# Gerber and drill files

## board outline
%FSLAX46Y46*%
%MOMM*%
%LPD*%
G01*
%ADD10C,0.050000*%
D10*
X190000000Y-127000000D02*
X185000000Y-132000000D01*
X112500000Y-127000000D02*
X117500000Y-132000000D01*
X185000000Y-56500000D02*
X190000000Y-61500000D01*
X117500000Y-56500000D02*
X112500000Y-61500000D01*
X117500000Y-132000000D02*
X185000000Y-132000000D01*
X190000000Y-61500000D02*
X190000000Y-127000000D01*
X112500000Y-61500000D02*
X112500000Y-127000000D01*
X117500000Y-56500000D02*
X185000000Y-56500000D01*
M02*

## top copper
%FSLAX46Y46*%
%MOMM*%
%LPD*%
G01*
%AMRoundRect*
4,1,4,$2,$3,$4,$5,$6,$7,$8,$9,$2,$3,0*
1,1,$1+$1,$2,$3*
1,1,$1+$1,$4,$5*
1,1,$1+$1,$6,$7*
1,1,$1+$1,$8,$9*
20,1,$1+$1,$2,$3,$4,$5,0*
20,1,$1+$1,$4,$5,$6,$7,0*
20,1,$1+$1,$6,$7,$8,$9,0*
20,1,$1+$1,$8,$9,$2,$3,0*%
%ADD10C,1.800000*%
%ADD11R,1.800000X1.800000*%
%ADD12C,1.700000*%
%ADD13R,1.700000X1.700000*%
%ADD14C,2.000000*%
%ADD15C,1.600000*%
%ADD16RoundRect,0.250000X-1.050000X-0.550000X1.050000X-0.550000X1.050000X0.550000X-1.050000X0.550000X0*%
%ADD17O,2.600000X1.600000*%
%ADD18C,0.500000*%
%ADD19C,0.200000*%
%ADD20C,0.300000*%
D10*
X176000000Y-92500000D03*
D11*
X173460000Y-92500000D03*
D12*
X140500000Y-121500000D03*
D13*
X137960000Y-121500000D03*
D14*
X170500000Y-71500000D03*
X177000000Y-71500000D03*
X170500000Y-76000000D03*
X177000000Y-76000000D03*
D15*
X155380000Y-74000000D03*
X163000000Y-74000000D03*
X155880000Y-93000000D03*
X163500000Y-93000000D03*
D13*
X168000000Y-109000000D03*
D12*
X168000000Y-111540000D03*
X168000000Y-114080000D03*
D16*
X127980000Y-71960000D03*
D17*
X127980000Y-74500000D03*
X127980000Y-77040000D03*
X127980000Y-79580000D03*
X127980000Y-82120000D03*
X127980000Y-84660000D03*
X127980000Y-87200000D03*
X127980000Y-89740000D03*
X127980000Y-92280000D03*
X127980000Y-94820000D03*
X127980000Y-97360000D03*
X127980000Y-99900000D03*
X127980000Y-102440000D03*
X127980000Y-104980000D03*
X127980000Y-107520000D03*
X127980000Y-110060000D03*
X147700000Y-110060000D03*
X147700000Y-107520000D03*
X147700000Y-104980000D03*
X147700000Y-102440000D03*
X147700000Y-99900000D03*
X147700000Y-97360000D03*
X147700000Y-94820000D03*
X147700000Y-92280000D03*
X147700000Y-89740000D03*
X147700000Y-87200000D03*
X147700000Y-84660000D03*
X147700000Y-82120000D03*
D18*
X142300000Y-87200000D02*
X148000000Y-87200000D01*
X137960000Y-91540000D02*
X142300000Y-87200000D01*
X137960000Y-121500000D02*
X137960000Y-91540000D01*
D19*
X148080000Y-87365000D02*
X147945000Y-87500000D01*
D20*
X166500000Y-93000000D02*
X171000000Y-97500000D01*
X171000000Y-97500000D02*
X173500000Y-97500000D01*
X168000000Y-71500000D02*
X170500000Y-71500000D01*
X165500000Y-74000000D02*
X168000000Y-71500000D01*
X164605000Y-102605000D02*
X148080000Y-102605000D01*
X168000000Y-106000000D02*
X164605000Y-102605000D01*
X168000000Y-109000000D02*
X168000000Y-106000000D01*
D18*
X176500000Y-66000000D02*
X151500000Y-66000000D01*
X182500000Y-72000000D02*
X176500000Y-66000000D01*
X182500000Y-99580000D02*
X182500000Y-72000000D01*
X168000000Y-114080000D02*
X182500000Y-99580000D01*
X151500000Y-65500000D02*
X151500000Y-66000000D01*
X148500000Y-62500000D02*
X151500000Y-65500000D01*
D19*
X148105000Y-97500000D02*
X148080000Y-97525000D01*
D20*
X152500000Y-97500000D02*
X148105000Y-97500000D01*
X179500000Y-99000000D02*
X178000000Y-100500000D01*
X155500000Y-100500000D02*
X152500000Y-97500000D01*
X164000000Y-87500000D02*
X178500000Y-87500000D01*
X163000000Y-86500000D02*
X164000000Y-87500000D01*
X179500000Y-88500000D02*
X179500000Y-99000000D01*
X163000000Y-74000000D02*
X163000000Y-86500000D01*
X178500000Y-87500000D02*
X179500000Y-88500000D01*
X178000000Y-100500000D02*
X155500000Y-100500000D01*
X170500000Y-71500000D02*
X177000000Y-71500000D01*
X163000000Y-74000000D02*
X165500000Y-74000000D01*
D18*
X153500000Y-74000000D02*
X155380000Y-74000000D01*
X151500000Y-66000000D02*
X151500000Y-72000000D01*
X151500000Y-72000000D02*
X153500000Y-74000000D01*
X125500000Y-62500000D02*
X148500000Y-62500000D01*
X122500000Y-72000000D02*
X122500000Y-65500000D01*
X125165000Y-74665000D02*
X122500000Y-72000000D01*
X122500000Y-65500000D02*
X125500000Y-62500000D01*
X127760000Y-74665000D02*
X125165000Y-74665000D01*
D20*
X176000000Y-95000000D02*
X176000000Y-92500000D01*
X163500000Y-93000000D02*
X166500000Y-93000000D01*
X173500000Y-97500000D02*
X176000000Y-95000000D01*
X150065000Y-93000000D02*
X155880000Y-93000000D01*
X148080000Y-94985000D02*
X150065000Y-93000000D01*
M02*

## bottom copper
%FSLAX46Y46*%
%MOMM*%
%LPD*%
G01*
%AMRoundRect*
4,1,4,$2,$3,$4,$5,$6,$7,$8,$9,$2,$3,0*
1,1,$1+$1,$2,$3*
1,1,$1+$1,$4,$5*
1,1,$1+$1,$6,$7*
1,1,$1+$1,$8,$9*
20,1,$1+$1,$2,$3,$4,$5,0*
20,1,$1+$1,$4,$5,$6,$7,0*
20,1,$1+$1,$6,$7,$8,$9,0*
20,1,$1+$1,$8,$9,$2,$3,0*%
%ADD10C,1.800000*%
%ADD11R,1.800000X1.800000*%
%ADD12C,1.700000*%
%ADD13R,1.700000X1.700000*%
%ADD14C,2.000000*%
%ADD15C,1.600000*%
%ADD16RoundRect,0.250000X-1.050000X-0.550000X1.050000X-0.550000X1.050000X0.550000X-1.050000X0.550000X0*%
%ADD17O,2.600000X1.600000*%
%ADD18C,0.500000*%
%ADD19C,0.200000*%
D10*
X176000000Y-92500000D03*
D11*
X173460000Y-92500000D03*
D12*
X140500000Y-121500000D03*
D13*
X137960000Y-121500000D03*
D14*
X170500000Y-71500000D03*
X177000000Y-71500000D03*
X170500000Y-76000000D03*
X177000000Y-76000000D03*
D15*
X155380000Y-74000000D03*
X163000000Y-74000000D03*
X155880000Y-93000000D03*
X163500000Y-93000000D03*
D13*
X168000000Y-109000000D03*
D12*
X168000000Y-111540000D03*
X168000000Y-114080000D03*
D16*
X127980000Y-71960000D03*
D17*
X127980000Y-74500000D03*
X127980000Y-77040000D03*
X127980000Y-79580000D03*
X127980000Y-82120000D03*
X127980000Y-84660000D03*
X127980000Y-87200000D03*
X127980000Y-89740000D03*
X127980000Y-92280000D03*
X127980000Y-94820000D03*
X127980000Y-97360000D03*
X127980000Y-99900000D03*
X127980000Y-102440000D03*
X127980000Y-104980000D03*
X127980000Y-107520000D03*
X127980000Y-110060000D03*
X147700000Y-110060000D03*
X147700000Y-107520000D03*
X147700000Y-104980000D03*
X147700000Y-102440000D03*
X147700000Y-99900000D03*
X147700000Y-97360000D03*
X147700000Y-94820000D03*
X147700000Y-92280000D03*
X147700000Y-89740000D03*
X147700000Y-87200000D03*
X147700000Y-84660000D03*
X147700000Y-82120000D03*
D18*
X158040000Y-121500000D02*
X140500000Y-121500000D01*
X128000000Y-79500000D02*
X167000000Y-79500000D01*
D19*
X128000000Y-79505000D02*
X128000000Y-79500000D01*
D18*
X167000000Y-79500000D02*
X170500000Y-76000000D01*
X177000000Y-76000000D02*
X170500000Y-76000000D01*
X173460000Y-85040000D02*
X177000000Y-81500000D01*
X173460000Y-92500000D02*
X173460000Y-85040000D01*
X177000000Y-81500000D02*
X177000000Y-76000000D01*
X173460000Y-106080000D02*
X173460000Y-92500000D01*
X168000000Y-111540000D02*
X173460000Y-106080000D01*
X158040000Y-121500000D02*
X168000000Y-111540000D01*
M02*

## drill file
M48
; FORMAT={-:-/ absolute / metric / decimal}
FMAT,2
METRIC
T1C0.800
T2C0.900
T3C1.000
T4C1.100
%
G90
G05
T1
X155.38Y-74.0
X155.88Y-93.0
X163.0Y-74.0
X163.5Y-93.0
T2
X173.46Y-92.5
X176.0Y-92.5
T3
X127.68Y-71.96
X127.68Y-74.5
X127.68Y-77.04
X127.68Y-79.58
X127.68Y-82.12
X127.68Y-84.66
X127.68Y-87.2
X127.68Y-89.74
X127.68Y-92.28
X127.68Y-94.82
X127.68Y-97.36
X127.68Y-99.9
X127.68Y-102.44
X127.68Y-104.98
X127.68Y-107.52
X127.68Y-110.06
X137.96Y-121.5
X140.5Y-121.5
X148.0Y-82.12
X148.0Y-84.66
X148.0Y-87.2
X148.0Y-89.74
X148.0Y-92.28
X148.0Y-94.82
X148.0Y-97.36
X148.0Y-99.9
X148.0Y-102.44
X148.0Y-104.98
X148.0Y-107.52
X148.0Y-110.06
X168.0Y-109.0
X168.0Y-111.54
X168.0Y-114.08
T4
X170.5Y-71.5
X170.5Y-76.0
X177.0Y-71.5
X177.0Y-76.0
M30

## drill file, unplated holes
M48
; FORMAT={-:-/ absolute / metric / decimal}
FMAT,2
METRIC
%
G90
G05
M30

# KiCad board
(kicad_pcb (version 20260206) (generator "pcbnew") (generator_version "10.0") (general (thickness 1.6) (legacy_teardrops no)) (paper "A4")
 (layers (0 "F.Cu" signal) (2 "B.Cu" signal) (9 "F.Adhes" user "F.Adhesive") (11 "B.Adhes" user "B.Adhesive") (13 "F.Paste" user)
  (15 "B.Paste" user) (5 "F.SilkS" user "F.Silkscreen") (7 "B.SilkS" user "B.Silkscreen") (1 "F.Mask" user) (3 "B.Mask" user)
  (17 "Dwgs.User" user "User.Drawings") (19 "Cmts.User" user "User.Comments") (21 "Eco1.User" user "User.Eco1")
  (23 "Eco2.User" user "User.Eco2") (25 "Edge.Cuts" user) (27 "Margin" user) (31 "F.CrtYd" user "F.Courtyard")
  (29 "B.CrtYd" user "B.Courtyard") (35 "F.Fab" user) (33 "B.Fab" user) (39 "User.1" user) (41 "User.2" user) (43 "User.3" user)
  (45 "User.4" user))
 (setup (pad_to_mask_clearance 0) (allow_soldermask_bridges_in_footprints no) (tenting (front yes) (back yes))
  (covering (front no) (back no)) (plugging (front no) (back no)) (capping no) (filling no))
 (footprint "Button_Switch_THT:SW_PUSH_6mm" (layer "F.Cu") (at 170.5 71.5)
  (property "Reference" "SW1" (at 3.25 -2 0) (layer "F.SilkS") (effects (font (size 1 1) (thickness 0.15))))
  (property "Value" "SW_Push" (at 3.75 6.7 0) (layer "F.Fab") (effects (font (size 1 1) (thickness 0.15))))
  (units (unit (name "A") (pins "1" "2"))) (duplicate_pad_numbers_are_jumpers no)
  (pad "1" thru_hole circle (at 0 0 90) (size 2 2) (drill 1.1) (layers "*.Cu" "*.Mask") (remove_unused_layers no)
   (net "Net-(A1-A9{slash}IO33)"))
  (pad "1" thru_hole circle (at 6.5 0 90) (size 2 2) (drill 1.1) (layers "*.Cu" "*.Mask") (remove_unused_layers no)
   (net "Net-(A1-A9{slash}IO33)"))
  (pad "2" thru_hole circle (at 0 4.5 90) (size 2 2) (drill 1.1) (layers "*.Cu" "*.Mask") (remove_unused_layers no) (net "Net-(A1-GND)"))
  (pad "2" thru_hole circle (at 6.5 4.5 90) (size 2 2) (drill 1.1) (layers "*.Cu" "*.Mask") (remove_unused_layers no) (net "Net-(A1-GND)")))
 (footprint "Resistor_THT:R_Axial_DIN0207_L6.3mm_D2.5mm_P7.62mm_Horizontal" (layer "F.Cu") (at 155.88 93)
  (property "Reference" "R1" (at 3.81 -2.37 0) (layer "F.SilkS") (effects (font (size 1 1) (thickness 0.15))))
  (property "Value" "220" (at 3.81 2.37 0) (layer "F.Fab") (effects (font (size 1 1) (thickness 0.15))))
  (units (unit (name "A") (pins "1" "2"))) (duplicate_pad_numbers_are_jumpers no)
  (pad "1" thru_hole circle (at 0 0) (size 1.6 1.6) (drill 0.8) (layers "*.Cu" "*.Mask") (remove_unused_layers no)
   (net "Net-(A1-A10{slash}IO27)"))
  (pad "2" thru_hole circle (at 7.62 0) (size 1.6 1.6) (drill 0.8) (layers "*.Cu" "*.Mask") (remove_unused_layers no) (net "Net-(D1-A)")))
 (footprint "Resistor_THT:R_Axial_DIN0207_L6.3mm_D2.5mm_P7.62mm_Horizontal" (layer "F.Cu") (at 155.38 74)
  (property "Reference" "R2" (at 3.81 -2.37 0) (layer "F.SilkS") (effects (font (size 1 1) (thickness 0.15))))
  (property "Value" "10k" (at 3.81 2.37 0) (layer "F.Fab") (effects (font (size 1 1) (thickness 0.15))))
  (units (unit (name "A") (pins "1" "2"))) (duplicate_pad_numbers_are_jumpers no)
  (pad "1" thru_hole circle (at 0 0) (size 1.6 1.6) (drill 0.8) (layers "*.Cu" "*.Mask") (remove_unused_layers no) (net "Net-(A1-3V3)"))
  (pad "2" thru_hole circle (at 7.62 0) (size 1.6 1.6) (drill 0.8) (layers "*.Cu" "*.Mask") (remove_unused_layers no)
   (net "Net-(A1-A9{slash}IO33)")))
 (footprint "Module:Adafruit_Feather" (layer "F.Cu") (at 127.68 71.96)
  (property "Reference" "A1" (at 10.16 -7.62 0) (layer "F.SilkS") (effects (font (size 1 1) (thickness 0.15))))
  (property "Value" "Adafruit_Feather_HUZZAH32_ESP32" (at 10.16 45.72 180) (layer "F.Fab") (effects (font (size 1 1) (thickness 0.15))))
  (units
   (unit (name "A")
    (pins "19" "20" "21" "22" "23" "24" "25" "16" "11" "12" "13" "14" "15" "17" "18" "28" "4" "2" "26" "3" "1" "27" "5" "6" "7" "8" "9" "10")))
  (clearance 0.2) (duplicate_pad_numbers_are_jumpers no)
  (pad "1" thru_hole roundrect (at 0 0) (size 2.6 1.6) (drill 1 (offset 0.3 0)) (layers "*.Cu" "*.Mask") (remove_unused_layers no)
   (roundrect_rratio 0.15625) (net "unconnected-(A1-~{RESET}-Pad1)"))
  (pad "2" thru_hole oval (at 0 2.54) (size 2.6 1.6) (drill 1 (offset 0.3 0)) (layers "*.Cu" "*.Mask") (remove_unused_layers no)
   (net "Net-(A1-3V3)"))
  (pad "3" thru_hole oval (at 0 5.08) (size 2.6 1.6) (drill 1 (offset 0.3 0)) (layers "*.Cu" "*.Mask") (remove_unused_layers no)
   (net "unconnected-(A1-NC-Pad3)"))
  (pad "4" thru_hole oval (at 0 7.62) (size 2.6 1.6) (drill 1 (offset 0.3 0)) (layers "*.Cu" "*.Mask") (remove_unused_layers no)
   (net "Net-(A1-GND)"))
  (pad "5" thru_hole oval (at 0 10.16) (size 2.6 1.6) (drill 1 (offset 0.3 0)) (layers "*.Cu" "*.Mask") (remove_unused_layers no)
   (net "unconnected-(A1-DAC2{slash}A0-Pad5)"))
  (pad "6" thru_hole oval (at 0 12.7) (size 2.6 1.6) (drill 1 (offset 0.3 0)) (layers "*.Cu" "*.Mask") (remove_unused_layers no)
   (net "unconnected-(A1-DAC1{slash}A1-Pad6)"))
  (pad "7" thru_hole oval (at 0 15.24) (size 2.6 1.6) (drill 1 (offset 0.3 0)) (layers "*.Cu" "*.Mask") (remove_unused_layers no)
   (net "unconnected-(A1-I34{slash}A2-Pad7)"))
  (pad "8" thru_hole oval (at 0 17.78) (size 2.6 1.6) (drill 1 (offset 0.3 0)) (layers "*.Cu" "*.Mask") (remove_unused_layers no)
   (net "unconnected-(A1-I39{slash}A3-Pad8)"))
  (pad "9" thru_hole oval (at 0 20.32) (size 2.6 1.6) (drill 1 (offset 0.3 0)) (layers "*.Cu" "*.Mask") (remove_unused_layers no)
   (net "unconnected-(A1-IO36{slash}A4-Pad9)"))
  (pad "10" thru_hole oval (at 0 22.86) (size 2.6 1.6) (drill 1 (offset 0.3 0)) (layers "*.Cu" "*.Mask") (remove_unused_layers no)
   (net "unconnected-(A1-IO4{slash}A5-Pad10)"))
  (pad "11" thru_hole oval (at 0 25.4) (size 2.6 1.6) (drill 1 (offset 0.3 0)) (layers "*.Cu" "*.Mask") (remove_unused_layers no)
   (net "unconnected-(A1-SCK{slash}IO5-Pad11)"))
  (pad "12" thru_hole oval (at 0 27.94) (size 2.6 1.6) (drill 1 (offset 0.3 0)) (layers "*.Cu" "*.Mask") (remove_unused_layers no)
   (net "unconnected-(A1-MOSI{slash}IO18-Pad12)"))
  (pad "13" thru_hole oval (at 0 30.48) (size 2.6 1.6) (drill 1 (offset 0.3 0)) (layers "*.Cu" "*.Mask") (remove_unused_layers no)
   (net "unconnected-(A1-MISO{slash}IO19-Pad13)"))
  (pad "14" thru_hole oval (at 0 33.02) (size 2.6 1.6) (drill 1 (offset 0.3 0)) (layers "*.Cu" "*.Mask") (remove_unused_layers no)
   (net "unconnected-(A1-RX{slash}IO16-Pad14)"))
  (pad "15" thru_hole oval (at 0 35.56) (size 2.6 1.6) (drill 1 (offset 0.3 0)) (layers "*.Cu" "*.Mask") (remove_unused_layers no)
   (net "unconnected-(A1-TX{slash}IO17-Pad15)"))
  (pad "16" thru_hole oval (at 0 38.1) (size 2.6 1.6) (drill 1 (offset 0.3 0)) (layers "*.Cu" "*.Mask") (remove_unused_layers no)
   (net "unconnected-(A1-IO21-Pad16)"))
  (pad "17" thru_hole oval (at 20.32 38.1 180) (size 2.6 1.6) (drill 1 (offset 0.3 0)) (layers "*.Cu" "*.Mask") (remove_unused_layers no)
   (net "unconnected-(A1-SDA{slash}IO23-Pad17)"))
  (pad "18" thru_hole oval (at 20.32 35.56 180) (size 2.6 1.6) (drill 1 (offset 0.3 0)) (layers "*.Cu" "*.Mask") (remove_unused_layers no)
   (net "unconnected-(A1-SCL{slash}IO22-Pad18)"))
  (pad "19" thru_hole oval (at 20.32 33.02 180) (size 2.6 1.6) (drill 1 (offset 0.3 0)) (layers "*.Cu" "*.Mask") (remove_unused_layers no)
   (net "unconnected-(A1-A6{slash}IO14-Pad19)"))
  (pad "20" thru_hole oval (at 20.32 30.48 180) (size 2.6 1.6) (drill 1 (offset 0.3 0)) (layers "*.Cu" "*.Mask") (remove_unused_layers no)
   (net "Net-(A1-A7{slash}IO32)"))
  (pad "21" thru_hole oval (at 20.32 27.94 180) (size 2.6 1.6) (drill 1 (offset 0.3 0)) (layers "*.Cu" "*.Mask") (remove_unused_layers no)
   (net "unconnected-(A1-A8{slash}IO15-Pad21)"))
  (pad "22" thru_hole oval (at 20.32 25.4 180) (size 2.6 1.6) (drill 1 (offset 0.3 0)) (layers "*.Cu" "*.Mask") (remove_unused_layers no)
   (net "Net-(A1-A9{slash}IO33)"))
  (pad "23" thru_hole oval (at 20.32 22.86 180) (size 2.6 1.6) (drill 1 (offset 0.3 0)) (layers "*.Cu" "*.Mask") (remove_unused_layers no)
   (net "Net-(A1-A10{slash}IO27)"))
  (pad "24" thru_hole oval (at 20.32 20.32 180) (size 2.6 1.6) (drill 1 (offset 0.3 0)) (layers "*.Cu" "*.Mask") (remove_unused_layers no)
   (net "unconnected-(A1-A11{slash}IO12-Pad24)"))
  (pad "25" thru_hole oval (at 20.32 17.78 180) (size 2.6 1.6) (drill 1 (offset 0.3 0)) (layers "*.Cu" "*.Mask") (remove_unused_layers no)
   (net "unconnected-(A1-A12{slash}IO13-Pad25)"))
  (pad "26" thru_hole oval (at 20.32 15.24 180) (size 2.6 1.6) (drill 1 (offset 0.3 0)) (layers "*.Cu" "*.Mask") (remove_unused_layers no)
   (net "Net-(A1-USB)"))
  (pad "27" thru_hole oval (at 20.32 12.7 180) (size 2.6 1.6) (drill 1 (offset 0.3 0)) (layers "*.Cu" "*.Mask") (remove_unused_layers no)
   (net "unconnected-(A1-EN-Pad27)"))
  (pad "28" thru_hole oval (at 20.32 10.16 180) (size 2.6 1.6) (drill 1 (offset 0.3 0)) (layers "*.Cu" "*.Mask") (remove_unused_layers no)
   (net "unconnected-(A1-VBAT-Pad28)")))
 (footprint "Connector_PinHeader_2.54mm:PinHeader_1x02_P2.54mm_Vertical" (layer "F.Cu") (at 137.96 121.5 90)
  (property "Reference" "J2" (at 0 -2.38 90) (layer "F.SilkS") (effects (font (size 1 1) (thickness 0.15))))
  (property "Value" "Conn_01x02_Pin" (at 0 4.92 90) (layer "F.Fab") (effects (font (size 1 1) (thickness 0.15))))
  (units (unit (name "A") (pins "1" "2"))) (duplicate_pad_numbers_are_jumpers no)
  (pad "1" thru_hole rect (at 0 0 90) (size 1.7 1.7) (drill 1) (layers "*.Cu" "*.Mask") (remove_unused_layers no) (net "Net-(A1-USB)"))
  (pad "2" thru_hole circle (at 0 2.54 90) (size 1.7 1.7) (drill 1) (layers "*.Cu" "*.Mask") (remove_unused_layers no) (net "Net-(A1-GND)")))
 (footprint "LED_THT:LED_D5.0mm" (layer "F.Cu") (at 173.46 92.5)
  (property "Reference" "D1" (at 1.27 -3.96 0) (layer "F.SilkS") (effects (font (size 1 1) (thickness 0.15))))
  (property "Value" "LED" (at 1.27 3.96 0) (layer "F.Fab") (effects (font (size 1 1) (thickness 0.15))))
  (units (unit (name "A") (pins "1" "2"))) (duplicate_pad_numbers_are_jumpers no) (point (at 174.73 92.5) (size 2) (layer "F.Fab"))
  (pad "1" thru_hole rect (at 0 0) (size 1.8 1.8) (drill 0.9) (layers "*.Cu" "*.Mask") (remove_unused_layers no) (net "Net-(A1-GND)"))
  (pad "2" thru_hole circle (at 2.54 0) (size 1.8 1.8) (drill 0.9) (layers "*.Cu" "*.Mask") (remove_unused_layers no) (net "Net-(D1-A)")))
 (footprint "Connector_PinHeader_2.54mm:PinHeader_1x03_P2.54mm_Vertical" (layer "F.Cu") (at 168 109)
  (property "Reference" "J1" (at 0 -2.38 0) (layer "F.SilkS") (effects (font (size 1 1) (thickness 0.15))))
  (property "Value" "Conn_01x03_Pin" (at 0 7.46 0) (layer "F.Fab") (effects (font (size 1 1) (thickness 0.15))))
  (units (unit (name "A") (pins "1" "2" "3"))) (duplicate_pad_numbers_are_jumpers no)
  (pad "1" thru_hole rect (at 0 0) (size 1.7 1.7) (drill 1) (layers "*.Cu" "*.Mask") (remove_unused_layers no)
   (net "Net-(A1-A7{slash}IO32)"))
  (pad "2" thru_hole circle (at 0 2.54) (size 1.7 1.7) (drill 1) (layers "*.Cu" "*.Mask") (remove_unused_layers no) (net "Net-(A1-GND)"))
  (pad "3" thru_hole circle (at 0 5.08) (size 1.7 1.7) (drill 1) (layers "*.Cu" "*.Mask") (remove_unused_layers no) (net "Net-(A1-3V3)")))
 (gr_line (start 112.5 61.5) (end 112.5 127) (stroke (width 0.05) (type default)) (layer "Edge.Cuts"))
 (gr_line (start 112.5 127) (end 117.5 132) (stroke (width 0.05) (type default)) (layer "Edge.Cuts"))
 (gr_line (start 117.5 56.5) (end 112.5 61.5) (stroke (width 0.05) (type default)) (layer "Edge.Cuts"))
 (gr_line (start 117.5 56.5) (end 185 56.5) (stroke (width 0.05) (type default)) (layer "Edge.Cuts"))
 (gr_line (start 117.5 132) (end 185 132) (stroke (width 0.05) (type default)) (layer "Edge.Cuts"))
 (gr_line (start 185 56.5) (end 190 61.5) (stroke (width 0.05) (type default)) (layer "Edge.Cuts"))
 (gr_line (start 190 61.5) (end 190 127) (stroke (width 0.05) (type default)) (layer "Edge.Cuts"))
 (gr_line (start 190 127) (end 185 132) (stroke (width 0.05) (type default)) (layer "Edge.Cuts"))
 (segment (start 148.08 94.985) (end 150.065 93) (width 0.3) (layer "F.Cu") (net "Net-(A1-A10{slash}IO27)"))
 (segment (start 150.065 93) (end 155.88 93) (width 0.3) (layer "F.Cu") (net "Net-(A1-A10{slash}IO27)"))
 (segment (start 173.46 92.5) (end 173.46 85.04) (width 0.5) (layer "B.Cu") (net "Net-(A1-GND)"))
 (segment (start 173.46 106.08) (end 173.46 92.5) (width 0.5) (layer "B.Cu") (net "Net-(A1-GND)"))
 (segment (start 158.04 121.5) (end 140.5 121.5) (width 0.5) (layer "B.Cu") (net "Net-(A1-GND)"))
 (segment (start 173.46 85.04) (end 177 81.5) (width 0.5) (layer "B.Cu") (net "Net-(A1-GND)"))
 (segment (start 167 79.5) (end 170.5 76) (width 0.5) (layer "B.Cu") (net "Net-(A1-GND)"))
 (segment (start 128 79.5) (end 167 79.5) (width 0.5) (layer "B.Cu") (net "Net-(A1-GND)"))
 (segment (start 168 111.54) (end 173.46 106.08) (width 0.5) (layer "B.Cu") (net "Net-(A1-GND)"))
 (segment (start 158.04 121.5) (end 168 111.54) (width 0.5) (layer "B.Cu") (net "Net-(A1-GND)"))
 (segment (start 177 76) (end 170.5 76) (width 0.5) (layer "B.Cu") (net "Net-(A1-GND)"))
 (segment (start 177 81.5) (end 177 76) (width 0.5) (layer "B.Cu") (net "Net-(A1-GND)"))
 (segment (start 128 79.505) (end 128 79.5) (width 0.2) (layer "B.Cu") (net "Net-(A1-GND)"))
 (segment (start 168 109) (end 168 106) (width 0.3) (layer "F.Cu") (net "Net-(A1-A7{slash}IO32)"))
 (segment (start 168 106) (end 164.605 102.605) (width 0.3) (layer "F.Cu") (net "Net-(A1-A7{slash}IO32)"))
 (segment (start 164.605 102.605) (end 148.08 102.605) (width 0.3) (layer "F.Cu") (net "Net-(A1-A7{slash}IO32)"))
 (segment (start 152.5 97.5) (end 148.105 97.5) (width 0.3) (layer "F.Cu") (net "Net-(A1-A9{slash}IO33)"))
 (segment (start 179.5 88.5) (end 179.5 99) (width 0.3) (layer "F.Cu") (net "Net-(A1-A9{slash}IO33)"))
 (segment (start 155.5 100.5) (end 152.5 97.5) (width 0.3) (layer "F.Cu") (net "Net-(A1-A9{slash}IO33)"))
 (segment (start 165.5 74) (end 168 71.5) (width 0.3) (layer "F.Cu") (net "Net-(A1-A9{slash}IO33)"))
 (segment (start 164 87.5) (end 178.5 87.5) (width 0.3) (layer "F.Cu") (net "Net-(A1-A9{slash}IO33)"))
 (segment (start 179.5 99) (end 178 100.5) (width 0.3) (layer "F.Cu") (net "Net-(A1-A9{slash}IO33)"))
 (segment (start 163 74) (end 163 86.5) (width 0.3) (layer "F.Cu") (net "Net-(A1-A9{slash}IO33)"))
 (segment (start 170.5 71.5) (end 177 71.5) (width 0.3) (layer "F.Cu") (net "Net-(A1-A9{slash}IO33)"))
 (segment (start 163 74) (end 165.5 74) (width 0.3) (layer "F.Cu") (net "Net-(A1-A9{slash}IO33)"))
 (segment (start 178 100.5) (end 155.5 100.5) (width 0.3) (layer "F.Cu") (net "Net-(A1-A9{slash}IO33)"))
 (segment (start 178.5 87.5) (end 179.5 88.5) (width 0.3) (layer "F.Cu") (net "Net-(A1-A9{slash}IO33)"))
 (segment (start 168 71.5) (end 170.5 71.5) (width 0.3) (layer "F.Cu") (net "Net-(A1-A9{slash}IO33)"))
 (segment (start 163 86.5) (end 164 87.5) (width 0.3) (layer "F.Cu") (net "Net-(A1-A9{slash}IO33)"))
 (segment (start 148.105 97.5) (end 148.08 97.525) (width 0.2) (layer "F.Cu") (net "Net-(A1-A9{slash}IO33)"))
 (segment (start 153.5 74) (end 155.38 74) (width 0.5) (layer "F.Cu") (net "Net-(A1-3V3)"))
 (segment (start 125.165 74.665) (end 122.5 72) (width 0.5) (layer "F.Cu") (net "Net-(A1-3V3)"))
 (segment (start 148.5 62.5) (end 151.5 65.5) (width 0.5) (layer "F.Cu") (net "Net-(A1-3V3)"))
 (segment (start 182.5 99.58) (end 182.5 72) (width 0.5) (layer "F.Cu") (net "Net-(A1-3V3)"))
 (segment (start 122.5 65.5) (end 125.5 62.5) (width 0.5) (layer "F.Cu") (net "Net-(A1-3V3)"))
 (segment (start 182.5 72) (end 176.5 66) (width 0.5) (layer "F.Cu") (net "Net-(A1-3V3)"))
 (segment (start 151.5 66) (end 151.5 72) (width 0.5) (layer "F.Cu") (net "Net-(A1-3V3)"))
 (segment (start 125.5 62.5) (end 148.5 62.5) (width 0.5) (layer "F.Cu") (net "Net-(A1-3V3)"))
 (segment (start 151.5 72) (end 153.5 74) (width 0.5) (layer "F.Cu") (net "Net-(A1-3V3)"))
 (segment (start 176.5 66) (end 151.5 66) (width 0.5) (layer "F.Cu") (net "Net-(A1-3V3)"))
 (segment (start 168 114.08) (end 182.5 99.58) (width 0.5) (layer "F.Cu") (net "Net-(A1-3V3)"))
 (segment (start 151.5 65.5) (end 151.5 66) (width 0.5) (layer "F.Cu") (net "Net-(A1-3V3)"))
 (segment (start 127.76 74.665) (end 125.165 74.665) (width 0.5) (layer "F.Cu") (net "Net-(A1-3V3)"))
 (segment (start 122.5 72) (end 122.5 65.5) (width 0.5) (layer "F.Cu") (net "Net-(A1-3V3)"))
 (segment (start 148.08 87.365) (end 147.945 87.5) (width 0.2) (layer "F.Cu") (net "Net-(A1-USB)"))
 (segment (start 137.96 121.5) (end 137.96 91.54) (width 0.5) (layer "F.Cu") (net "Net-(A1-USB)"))
 (segment (start 137.96 91.54) (end 142.3 87.2) (width 0.5) (layer "F.Cu") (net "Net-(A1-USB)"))
 (segment (start 142.3 87.2) (end 148 87.2) (width 0.5) (layer "F.Cu") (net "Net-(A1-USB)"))
 (segment (start 171 97.5) (end 173.5 97.5) (width 0.3) (layer "F.Cu") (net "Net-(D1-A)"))
 (segment (start 166.5 93) (end 171 97.5) (width 0.3) (layer "F.Cu") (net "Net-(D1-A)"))
 (segment (start 176 95) (end 176 92.5) (width 0.3) (layer "F.Cu") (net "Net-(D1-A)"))
 (segment (start 173.5 97.5) (end 176 95) (width 0.3) (layer "F.Cu") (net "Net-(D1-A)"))
 (segment (start 163.5 93) (end 166.5 93) (width 0.3) (layer "F.Cu") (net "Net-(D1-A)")))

